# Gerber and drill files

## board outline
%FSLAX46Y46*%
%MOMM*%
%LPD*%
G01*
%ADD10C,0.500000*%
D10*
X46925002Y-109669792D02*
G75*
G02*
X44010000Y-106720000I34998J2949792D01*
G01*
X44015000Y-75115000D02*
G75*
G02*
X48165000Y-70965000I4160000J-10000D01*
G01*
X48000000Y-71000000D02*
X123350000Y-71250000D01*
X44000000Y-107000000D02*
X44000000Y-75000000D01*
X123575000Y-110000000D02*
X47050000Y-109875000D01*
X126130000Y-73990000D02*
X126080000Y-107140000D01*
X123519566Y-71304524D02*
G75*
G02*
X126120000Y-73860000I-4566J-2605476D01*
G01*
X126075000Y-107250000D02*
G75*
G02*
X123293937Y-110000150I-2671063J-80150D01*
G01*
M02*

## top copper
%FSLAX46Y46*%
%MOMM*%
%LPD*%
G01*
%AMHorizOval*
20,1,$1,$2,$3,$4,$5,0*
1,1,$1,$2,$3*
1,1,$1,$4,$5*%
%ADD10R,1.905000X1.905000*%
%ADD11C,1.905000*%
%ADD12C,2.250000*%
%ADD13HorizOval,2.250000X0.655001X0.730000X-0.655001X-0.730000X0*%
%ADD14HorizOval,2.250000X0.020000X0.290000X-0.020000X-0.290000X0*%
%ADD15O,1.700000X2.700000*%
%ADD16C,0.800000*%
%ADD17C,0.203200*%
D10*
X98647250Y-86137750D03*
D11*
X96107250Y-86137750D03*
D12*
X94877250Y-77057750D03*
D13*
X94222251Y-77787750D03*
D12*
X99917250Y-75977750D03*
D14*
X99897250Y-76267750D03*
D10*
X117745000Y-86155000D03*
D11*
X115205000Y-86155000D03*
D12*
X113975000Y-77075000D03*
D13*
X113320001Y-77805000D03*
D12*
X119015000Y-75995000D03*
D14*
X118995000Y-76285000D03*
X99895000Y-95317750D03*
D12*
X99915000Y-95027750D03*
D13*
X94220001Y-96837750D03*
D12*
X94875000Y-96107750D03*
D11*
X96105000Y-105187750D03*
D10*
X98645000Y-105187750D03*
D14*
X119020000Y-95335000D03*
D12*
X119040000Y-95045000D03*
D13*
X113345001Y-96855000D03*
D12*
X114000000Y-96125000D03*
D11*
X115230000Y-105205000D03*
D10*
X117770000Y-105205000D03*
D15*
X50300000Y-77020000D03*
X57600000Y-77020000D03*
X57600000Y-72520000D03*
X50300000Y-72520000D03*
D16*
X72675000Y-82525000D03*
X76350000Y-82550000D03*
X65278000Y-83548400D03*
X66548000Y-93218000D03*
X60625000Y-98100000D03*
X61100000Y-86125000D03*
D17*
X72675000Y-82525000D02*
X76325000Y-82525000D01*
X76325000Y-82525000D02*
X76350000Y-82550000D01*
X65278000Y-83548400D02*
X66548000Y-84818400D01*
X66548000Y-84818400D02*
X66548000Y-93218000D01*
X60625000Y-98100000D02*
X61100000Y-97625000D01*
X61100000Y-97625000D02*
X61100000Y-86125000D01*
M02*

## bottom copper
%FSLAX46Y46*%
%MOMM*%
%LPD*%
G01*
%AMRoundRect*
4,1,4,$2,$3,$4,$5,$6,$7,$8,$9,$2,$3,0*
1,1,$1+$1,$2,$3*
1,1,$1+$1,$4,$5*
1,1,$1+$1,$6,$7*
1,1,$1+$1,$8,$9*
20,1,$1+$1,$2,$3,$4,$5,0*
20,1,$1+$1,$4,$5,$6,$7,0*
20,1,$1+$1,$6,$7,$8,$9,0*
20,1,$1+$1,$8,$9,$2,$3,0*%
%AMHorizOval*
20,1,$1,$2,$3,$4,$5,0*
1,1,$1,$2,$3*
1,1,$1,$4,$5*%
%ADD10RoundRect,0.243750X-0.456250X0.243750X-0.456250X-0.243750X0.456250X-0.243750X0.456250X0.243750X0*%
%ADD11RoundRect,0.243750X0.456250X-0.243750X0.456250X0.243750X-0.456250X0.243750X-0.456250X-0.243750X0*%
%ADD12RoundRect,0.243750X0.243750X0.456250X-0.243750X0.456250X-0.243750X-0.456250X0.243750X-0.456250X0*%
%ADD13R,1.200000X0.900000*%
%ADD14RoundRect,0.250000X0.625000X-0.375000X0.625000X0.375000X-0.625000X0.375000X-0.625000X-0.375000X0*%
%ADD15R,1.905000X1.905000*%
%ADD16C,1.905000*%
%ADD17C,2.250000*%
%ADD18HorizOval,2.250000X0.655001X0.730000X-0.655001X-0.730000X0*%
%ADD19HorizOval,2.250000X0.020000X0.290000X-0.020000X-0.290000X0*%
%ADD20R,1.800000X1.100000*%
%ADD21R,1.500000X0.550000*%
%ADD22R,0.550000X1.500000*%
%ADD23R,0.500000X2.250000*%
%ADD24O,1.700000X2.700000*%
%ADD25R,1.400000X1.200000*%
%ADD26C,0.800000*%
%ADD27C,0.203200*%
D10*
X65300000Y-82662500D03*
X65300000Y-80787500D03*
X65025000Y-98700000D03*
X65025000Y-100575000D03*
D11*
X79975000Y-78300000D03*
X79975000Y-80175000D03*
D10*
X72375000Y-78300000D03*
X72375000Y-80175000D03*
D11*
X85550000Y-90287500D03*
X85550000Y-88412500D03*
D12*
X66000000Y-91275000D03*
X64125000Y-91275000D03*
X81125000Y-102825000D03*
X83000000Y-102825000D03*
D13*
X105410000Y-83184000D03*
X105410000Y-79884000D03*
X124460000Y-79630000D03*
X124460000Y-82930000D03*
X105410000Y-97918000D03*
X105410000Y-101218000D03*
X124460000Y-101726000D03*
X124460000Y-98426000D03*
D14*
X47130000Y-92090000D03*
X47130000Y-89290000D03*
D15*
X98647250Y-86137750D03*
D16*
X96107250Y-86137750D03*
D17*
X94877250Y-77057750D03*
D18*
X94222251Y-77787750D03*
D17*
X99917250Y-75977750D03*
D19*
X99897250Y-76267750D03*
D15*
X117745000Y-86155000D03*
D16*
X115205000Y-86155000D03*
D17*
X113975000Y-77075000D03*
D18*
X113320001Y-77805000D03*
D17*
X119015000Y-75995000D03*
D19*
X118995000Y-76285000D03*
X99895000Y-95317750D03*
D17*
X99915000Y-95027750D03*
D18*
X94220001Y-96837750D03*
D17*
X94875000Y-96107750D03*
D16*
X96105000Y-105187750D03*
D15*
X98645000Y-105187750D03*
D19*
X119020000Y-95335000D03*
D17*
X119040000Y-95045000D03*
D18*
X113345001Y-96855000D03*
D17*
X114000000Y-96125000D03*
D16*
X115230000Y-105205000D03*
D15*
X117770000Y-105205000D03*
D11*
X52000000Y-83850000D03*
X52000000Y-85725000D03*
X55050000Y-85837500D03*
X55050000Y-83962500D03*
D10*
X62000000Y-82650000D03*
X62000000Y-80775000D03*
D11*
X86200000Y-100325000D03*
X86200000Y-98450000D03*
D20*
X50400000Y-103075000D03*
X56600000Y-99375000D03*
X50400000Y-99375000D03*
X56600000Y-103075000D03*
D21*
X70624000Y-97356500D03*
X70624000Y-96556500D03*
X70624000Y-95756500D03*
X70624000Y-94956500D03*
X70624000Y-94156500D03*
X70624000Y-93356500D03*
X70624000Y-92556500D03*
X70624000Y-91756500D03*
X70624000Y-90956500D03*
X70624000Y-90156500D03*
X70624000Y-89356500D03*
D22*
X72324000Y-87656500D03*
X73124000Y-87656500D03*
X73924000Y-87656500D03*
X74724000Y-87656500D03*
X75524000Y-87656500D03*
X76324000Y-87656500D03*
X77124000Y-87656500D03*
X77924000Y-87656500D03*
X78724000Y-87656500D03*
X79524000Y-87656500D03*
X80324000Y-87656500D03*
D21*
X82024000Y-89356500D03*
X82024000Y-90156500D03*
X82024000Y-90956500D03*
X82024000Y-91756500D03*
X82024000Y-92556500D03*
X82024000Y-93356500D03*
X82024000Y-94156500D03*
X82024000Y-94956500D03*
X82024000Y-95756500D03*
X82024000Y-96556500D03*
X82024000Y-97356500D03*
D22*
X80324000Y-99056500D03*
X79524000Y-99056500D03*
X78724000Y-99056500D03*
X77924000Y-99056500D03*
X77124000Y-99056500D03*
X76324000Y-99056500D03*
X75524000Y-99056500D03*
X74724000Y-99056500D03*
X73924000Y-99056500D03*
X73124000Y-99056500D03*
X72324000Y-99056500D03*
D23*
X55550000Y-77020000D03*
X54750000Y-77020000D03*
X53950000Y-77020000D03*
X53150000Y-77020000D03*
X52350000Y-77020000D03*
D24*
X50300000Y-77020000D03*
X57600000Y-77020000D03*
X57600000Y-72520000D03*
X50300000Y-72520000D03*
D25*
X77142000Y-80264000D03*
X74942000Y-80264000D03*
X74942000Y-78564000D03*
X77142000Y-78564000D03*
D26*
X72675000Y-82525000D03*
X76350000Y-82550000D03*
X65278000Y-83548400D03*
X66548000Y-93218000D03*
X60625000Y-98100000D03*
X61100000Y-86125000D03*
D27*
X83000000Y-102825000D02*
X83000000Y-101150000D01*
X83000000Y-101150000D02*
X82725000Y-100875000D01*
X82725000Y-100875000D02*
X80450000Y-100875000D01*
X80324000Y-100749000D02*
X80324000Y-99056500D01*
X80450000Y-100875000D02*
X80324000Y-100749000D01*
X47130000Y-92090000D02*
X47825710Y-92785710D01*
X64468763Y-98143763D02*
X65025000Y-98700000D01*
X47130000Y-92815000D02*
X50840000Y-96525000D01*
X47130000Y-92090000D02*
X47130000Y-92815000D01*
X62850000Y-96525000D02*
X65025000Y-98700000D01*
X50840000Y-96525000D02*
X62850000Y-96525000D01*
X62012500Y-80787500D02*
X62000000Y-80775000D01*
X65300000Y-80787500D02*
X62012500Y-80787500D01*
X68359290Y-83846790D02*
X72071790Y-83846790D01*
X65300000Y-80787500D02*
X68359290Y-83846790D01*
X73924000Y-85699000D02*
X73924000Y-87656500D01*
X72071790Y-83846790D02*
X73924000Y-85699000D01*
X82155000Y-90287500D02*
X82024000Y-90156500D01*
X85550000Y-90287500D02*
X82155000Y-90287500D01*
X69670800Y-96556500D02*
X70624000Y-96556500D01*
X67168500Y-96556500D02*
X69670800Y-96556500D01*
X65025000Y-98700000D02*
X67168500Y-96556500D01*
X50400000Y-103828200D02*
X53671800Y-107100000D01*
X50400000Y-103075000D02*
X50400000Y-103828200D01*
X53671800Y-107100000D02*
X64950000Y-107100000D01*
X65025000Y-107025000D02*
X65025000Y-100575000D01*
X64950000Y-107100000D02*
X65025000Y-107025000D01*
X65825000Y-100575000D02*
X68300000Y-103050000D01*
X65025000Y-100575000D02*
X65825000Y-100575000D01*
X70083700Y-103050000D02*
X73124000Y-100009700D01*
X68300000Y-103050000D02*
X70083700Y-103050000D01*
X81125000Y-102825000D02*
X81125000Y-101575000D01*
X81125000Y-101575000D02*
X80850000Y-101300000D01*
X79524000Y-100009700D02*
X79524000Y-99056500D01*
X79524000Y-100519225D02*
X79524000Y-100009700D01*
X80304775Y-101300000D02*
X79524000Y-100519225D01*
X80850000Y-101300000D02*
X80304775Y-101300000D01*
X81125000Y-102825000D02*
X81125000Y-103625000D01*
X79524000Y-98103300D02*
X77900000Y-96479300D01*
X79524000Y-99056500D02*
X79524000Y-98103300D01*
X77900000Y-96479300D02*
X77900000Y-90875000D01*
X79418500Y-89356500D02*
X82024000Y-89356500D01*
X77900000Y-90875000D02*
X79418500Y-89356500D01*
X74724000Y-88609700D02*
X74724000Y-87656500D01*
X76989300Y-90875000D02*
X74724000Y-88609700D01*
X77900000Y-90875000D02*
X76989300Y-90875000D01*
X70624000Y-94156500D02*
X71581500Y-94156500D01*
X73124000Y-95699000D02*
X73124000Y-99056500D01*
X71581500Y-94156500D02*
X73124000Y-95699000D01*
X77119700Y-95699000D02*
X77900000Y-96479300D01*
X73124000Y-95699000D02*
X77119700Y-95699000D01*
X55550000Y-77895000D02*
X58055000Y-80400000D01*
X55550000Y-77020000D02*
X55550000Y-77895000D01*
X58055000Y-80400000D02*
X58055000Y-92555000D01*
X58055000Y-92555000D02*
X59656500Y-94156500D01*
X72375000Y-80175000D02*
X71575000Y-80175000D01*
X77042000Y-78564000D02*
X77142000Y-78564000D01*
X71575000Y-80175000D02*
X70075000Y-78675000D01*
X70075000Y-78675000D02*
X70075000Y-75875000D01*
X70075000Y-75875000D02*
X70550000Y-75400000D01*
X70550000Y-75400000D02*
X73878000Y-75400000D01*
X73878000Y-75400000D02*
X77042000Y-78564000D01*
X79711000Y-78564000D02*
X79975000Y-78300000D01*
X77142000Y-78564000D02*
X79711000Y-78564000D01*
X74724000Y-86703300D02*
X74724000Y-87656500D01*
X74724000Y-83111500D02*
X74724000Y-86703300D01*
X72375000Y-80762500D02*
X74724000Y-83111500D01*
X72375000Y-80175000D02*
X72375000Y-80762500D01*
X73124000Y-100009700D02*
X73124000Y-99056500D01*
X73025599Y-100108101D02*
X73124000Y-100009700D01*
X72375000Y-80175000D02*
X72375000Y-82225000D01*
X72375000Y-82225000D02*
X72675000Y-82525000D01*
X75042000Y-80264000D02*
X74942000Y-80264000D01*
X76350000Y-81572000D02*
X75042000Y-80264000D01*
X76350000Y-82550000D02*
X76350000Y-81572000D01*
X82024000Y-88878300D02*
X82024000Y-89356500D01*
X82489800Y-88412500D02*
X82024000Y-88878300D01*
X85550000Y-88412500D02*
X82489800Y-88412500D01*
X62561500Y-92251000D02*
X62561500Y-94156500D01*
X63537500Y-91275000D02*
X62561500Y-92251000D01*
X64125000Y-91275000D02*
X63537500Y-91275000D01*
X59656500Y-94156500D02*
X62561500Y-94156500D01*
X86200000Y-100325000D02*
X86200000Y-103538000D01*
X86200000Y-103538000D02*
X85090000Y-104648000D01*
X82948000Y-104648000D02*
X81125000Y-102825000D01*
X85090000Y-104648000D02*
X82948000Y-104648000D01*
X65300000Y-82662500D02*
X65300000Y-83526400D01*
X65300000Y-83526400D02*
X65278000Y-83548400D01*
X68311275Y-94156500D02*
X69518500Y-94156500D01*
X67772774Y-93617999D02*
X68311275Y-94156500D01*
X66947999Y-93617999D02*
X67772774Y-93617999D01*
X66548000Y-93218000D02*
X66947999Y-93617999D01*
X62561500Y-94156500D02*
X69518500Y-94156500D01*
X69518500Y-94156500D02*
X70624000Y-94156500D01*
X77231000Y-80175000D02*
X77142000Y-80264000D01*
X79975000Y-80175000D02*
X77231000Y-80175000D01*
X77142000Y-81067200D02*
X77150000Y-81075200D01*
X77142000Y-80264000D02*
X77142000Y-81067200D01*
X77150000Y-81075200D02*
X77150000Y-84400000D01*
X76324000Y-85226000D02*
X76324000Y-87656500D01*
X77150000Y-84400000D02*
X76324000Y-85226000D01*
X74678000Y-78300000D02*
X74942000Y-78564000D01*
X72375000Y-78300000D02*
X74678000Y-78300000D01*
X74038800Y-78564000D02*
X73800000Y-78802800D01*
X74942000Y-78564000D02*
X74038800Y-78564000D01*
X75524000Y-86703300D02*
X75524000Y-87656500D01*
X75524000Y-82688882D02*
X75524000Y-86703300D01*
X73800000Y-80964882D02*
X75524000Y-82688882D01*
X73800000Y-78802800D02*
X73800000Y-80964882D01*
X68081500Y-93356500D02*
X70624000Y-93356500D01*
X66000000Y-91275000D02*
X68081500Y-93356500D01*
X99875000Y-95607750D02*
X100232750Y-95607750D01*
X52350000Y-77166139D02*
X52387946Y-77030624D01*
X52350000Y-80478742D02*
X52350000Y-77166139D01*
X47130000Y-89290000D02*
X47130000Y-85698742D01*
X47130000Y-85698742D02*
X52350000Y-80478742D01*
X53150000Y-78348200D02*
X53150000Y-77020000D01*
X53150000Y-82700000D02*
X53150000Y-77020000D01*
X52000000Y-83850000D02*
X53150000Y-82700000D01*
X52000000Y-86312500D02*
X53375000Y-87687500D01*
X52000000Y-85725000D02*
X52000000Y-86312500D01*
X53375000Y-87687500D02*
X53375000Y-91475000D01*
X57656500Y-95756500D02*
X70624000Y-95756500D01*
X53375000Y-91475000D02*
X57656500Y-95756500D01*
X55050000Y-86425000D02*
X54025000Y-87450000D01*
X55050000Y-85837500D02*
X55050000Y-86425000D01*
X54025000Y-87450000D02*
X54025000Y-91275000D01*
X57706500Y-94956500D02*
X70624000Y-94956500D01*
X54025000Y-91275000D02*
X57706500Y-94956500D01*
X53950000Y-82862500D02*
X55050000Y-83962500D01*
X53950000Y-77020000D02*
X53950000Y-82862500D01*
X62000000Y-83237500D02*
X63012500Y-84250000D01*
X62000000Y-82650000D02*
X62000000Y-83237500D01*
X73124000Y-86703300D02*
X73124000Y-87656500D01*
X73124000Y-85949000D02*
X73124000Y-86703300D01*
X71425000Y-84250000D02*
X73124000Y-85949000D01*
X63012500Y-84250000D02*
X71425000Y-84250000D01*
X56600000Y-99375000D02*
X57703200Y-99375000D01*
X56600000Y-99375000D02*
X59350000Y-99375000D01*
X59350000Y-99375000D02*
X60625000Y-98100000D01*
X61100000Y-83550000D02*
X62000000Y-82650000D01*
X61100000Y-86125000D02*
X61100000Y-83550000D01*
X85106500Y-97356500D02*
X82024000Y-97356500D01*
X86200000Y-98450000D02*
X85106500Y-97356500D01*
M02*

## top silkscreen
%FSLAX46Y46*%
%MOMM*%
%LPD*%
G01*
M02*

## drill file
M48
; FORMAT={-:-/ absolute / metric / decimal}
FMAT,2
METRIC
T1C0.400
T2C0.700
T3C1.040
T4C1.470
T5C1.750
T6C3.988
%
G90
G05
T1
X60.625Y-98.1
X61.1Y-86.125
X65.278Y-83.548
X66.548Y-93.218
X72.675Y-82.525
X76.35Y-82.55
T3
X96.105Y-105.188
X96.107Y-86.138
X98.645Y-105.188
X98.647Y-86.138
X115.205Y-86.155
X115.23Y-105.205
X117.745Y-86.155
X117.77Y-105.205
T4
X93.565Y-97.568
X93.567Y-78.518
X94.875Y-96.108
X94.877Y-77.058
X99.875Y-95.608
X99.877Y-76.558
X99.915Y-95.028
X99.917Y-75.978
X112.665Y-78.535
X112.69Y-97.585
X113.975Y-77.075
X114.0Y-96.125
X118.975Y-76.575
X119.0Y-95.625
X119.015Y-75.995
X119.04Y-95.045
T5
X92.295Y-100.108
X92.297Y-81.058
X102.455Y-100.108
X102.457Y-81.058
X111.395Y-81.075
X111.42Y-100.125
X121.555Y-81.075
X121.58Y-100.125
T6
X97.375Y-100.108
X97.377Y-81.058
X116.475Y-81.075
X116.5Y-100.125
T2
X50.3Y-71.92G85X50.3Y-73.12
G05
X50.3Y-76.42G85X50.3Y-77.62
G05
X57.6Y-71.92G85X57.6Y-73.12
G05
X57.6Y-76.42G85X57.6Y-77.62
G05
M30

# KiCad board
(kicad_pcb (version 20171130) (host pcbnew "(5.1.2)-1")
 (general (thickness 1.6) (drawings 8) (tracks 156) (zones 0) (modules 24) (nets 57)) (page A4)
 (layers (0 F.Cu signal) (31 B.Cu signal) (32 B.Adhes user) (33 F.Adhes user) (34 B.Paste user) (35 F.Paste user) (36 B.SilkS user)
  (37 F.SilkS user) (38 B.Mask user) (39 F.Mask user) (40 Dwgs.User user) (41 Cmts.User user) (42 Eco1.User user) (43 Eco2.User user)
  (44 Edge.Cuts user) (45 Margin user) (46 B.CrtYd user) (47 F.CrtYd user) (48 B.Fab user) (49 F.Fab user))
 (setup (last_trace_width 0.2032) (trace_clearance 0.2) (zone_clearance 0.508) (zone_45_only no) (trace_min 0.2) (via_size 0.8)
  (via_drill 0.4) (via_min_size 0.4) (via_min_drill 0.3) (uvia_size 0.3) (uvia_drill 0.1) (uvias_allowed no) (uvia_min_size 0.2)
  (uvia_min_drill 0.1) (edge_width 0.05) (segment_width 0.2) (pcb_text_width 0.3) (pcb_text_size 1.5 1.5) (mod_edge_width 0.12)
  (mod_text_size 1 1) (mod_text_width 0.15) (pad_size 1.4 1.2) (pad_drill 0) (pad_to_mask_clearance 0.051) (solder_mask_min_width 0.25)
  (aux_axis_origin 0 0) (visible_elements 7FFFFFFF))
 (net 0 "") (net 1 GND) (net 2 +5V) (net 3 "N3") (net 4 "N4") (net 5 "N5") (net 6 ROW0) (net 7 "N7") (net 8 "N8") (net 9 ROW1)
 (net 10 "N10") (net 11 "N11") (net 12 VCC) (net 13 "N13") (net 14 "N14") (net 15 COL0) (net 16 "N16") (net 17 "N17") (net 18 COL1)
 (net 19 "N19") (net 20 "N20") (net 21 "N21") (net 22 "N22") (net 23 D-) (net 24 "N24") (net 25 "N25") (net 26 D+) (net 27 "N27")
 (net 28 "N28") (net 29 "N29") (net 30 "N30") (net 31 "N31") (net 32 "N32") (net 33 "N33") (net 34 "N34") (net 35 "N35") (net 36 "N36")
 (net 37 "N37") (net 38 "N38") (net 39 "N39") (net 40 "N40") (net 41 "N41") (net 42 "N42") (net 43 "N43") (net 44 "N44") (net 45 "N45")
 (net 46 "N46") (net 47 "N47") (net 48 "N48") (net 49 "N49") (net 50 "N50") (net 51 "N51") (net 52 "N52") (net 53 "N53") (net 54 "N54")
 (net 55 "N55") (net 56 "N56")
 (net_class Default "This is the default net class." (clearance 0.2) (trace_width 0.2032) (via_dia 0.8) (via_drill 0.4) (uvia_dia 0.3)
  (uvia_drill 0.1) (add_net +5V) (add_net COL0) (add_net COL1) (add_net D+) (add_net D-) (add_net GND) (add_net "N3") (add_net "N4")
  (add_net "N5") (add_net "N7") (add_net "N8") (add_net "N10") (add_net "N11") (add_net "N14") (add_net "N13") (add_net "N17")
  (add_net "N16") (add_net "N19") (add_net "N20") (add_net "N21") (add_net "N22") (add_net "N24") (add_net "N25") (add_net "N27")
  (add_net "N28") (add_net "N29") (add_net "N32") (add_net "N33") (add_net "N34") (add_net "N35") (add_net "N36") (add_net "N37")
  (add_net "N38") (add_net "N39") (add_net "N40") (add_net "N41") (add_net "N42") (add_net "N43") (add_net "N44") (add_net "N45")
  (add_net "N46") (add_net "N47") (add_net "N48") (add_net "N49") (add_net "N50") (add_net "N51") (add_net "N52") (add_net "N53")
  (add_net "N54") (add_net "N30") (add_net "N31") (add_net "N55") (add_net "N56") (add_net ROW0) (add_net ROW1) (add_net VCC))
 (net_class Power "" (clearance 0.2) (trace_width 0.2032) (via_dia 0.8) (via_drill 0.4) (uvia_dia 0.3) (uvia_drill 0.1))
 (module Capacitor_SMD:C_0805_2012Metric (layer B.Cu) (at 65.3 81.725 270)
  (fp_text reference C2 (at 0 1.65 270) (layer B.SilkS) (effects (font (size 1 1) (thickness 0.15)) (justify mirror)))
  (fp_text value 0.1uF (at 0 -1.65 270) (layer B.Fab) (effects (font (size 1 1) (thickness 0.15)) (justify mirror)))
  (pad 2 smd roundrect (at 0.9375 0 270) (size 0.975 1.4) (layers B.Cu B.Paste B.Mask) (roundrect_rratio 0.25) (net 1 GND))
  (pad 1 smd roundrect (at -0.9375 0 270) (size 0.975 1.4) (layers B.Cu B.Paste B.Mask) (roundrect_rratio 0.25) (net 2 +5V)))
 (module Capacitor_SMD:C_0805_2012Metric (layer B.Cu) (at 65.025 99.6375 270)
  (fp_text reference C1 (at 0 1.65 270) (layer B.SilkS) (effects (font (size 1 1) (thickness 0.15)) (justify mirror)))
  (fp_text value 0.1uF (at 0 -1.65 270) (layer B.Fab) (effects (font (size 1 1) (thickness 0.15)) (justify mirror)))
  (pad 1 smd roundrect (at -0.9375 0 270) (size 0.975 1.4) (layers B.Cu B.Paste B.Mask) (roundrect_rratio 0.25) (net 2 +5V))
  (pad 2 smd roundrect (at 0.9375 0 270) (size 0.975 1.4) (layers B.Cu B.Paste B.Mask) (roundrect_rratio 0.25) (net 1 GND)))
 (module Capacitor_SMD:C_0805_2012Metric (layer B.Cu) (at 79.975 79.2375 90)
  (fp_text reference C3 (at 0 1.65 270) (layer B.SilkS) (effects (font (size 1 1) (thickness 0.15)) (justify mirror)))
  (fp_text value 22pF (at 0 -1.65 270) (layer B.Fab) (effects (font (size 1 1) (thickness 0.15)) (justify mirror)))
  (pad 2 smd roundrect (at 0.9375 0 90) (size 0.975 1.4) (layers B.Cu B.Paste B.Mask) (roundrect_rratio 0.25) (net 1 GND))
  (pad 1 smd roundrect (at -0.9375 0 90) (size 0.975 1.4) (layers B.Cu B.Paste B.Mask) (roundrect_rratio 0.25) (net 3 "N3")))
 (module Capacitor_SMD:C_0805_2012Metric (layer B.Cu) (at 72.375 79.2375 270)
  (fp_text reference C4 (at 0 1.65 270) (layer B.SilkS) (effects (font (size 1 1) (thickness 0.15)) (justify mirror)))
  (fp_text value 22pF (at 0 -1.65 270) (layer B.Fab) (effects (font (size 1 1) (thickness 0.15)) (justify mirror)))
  (pad 1 smd roundrect (at -0.9375 0 270) (size 0.975 1.4) (layers B.Cu B.Paste B.Mask) (roundrect_rratio 0.25) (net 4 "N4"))
  (pad 2 smd roundrect (at 0.9375 0 270) (size 0.975 1.4) (layers B.Cu B.Paste B.Mask) (roundrect_rratio 0.25) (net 1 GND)))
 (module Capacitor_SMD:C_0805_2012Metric (layer B.Cu) (at 85.55 89.35 90)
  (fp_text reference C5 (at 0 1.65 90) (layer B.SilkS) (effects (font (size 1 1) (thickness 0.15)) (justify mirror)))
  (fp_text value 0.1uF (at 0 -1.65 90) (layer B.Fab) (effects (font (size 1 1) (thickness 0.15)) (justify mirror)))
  (pad 1 smd roundrect (at -0.9375 0 90) (size 0.975 1.4) (layers B.Cu B.Paste B.Mask) (roundrect_rratio 0.25) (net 2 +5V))
  (pad 2 smd roundrect (at 0.9375 0 90) (size 0.975 1.4) (layers B.Cu B.Paste B.Mask) (roundrect_rratio 0.25) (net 1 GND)))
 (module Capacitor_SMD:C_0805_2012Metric (layer B.Cu) (at 65.0625 91.275 180)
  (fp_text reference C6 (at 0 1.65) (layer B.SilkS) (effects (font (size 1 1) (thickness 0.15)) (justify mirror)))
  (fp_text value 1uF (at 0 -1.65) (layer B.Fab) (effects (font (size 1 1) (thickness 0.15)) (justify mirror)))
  (pad 1 smd roundrect (at -0.9375 0 180) (size 0.975 1.4) (layers B.Cu B.Paste B.Mask) (roundrect_rratio 0.25) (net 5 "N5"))
  (pad 2 smd roundrect (at 0.9375 0 180) (size 0.975 1.4) (layers B.Cu B.Paste B.Mask) (roundrect_rratio 0.25) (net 1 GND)))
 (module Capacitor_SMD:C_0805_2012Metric (layer B.Cu) (at 82.0625 102.825 180)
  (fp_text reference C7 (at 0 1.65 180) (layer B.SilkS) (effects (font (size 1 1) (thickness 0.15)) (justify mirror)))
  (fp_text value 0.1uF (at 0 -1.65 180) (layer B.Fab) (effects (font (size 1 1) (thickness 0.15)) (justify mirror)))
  (pad 2 smd roundrect (at 0.9375 0 180) (size 0.975 1.4) (layers B.Cu B.Paste B.Mask) (roundrect_rratio 0.25) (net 1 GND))
  (pad 1 smd roundrect (at -0.9375 0 180) (size 0.975 1.4) (layers B.Cu B.Paste B.Mask) (roundrect_rratio 0.25) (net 2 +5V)))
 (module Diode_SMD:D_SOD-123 (layer B.Cu) (at 105.41 81.534 90)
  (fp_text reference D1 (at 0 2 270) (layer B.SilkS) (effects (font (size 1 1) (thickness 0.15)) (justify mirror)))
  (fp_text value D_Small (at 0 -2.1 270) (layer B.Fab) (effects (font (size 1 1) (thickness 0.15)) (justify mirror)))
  (pad 1 smd rect (at -1.65 0 90) (size 0.9 1.2) (layers B.Cu B.Paste B.Mask) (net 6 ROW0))
  (pad 2 smd rect (at 1.65 0 90) (size 0.9 1.2) (layers B.Cu B.Paste B.Mask) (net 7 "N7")))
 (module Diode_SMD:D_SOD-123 (layer B.Cu) (at 124.46 81.28 90)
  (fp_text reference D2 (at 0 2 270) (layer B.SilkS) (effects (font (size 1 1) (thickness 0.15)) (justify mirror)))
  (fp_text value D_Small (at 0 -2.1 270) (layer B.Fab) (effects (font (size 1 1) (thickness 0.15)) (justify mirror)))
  (pad 2 smd rect (at 1.65 0 90) (size 0.9 1.2) (layers B.Cu B.Paste B.Mask) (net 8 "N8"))
  (pad 1 smd rect (at -1.65 0 90) (size 0.9 1.2) (layers B.Cu B.Paste B.Mask) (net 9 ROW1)))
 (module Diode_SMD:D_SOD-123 (layer B.Cu) (at 105.41 99.568 270)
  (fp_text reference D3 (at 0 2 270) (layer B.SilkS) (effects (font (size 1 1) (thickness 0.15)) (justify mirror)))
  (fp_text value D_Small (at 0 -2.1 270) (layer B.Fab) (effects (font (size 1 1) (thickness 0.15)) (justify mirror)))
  (pad 1 smd rect (at -1.65 0 270) (size 0.9 1.2) (layers B.Cu B.Paste B.Mask) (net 6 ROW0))
  (pad 2 smd rect (at 1.65 0 270) (size 0.9 1.2) (layers B.Cu B.Paste B.Mask) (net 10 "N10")))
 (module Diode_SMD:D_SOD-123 (layer B.Cu) (at 124.46 100.076 270)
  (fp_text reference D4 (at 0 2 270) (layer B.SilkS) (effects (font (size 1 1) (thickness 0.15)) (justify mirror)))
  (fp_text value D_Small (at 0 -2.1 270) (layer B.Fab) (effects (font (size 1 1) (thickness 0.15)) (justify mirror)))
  (pad 2 smd rect (at 1.65 0 270) (size 0.9 1.2) (layers B.Cu B.Paste B.Mask) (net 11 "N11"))
  (pad 1 smd rect (at -1.65 0 270) (size 0.9 1.2) (layers B.Cu B.Paste B.Mask) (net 9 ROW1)))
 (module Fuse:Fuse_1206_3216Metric (layer B.Cu) (at 47.13 90.69 90)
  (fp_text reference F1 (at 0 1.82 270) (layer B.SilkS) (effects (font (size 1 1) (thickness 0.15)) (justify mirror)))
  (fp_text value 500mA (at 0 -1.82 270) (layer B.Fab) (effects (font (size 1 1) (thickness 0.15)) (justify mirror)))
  (pad 1 smd roundrect (at -1.4 0 90) (size 1.25 1.75) (layers B.Cu B.Paste B.Mask) (roundrect_rratio 0.2) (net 2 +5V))
  (pad 2 smd roundrect (at 1.4 0 90) (size 1.25 1.75) (layers B.Cu B.Paste B.Mask) (roundrect_rratio 0.2) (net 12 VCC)))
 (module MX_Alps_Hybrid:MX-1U (layer F.Cu) (at 97.37725 81.05775)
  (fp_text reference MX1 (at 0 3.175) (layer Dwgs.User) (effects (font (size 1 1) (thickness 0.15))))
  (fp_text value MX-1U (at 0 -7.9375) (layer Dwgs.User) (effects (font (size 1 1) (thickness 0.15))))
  (pad "" np_thru_hole circle (at 5.08 0 48.0996) (size 1.75 1.75) (drill 1.75) (layers *.Cu *.Mask))
  (pad "" np_thru_hole circle (at -5.08 0 48.0996) (size 1.75 1.75) (drill 1.75) (layers *.Cu *.Mask))
  (pad 4 thru_hole rect (at 1.27 5.08) (size 1.905 1.905) (drill 1.04) (layers *.Cu B.Mask) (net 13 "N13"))
  (pad 3 thru_hole circle (at -1.27 5.08) (size 1.905 1.905) (drill 1.04) (layers *.Cu B.Mask) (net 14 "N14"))
  (pad 1 thru_hole circle (at -2.5 -4) (size 2.25 2.25) (drill 1.47) (layers *.Cu B.Mask) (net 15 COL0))
  (pad "" np_thru_hole circle (at 0 0) (size 3.9878 3.9878) (drill 3.9878) (layers *.Cu *.Mask))
  (pad 1 thru_hole oval (at -3.81 -2.54 48.0996) (size 4.211556 2.25) (drill 1.47 (offset 0.980778 0)) (layers *.Cu B.Mask) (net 15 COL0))
  (pad 2 thru_hole circle (at 2.54 -5.08) (size 2.25 2.25) (drill 1.47) (layers *.Cu B.Mask) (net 7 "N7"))
  (pad 2 thru_hole oval (at 2.5 -4.5 86.0548) (size 2.831378 2.25) (drill 1.47 (offset 0.290689 0)) (layers *.Cu B.Mask) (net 7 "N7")))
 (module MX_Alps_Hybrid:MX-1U (layer F.Cu) (at 116.475 81.075)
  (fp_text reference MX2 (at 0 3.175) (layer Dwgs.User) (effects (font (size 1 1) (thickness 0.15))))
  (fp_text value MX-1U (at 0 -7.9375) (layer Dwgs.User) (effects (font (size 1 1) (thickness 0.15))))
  (pad "" np_thru_hole circle (at 5.08 0 48.0996) (size 1.75 1.75) (drill 1.75) (layers *.Cu *.Mask))
  (pad "" np_thru_hole circle (at -5.08 0 48.0996) (size 1.75 1.75) (drill 1.75) (layers *.Cu *.Mask))
  (pad 4 thru_hole rect (at 1.27 5.08) (size 1.905 1.905) (drill 1.04) (layers *.Cu B.Mask) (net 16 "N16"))
  (pad 3 thru_hole circle (at -1.27 5.08) (size 1.905 1.905) (drill 1.04) (layers *.Cu B.Mask) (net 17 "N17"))
  (pad 1 thru_hole circle (at -2.5 -4) (size 2.25 2.25) (drill 1.47) (layers *.Cu B.Mask) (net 15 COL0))
  (pad "" np_thru_hole circle (at 0 0) (size 3.9878 3.9878) (drill 3.9878) (layers *.Cu *.Mask))
  (pad 1 thru_hole oval (at -3.81 -2.54 48.0996) (size 4.211556 2.25) (drill 1.47 (offset 0.980778 0)) (layers *.Cu B.Mask) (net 15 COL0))
  (pad 2 thru_hole circle (at 2.54 -5.08) (size 2.25 2.25) (drill 1.47) (layers *.Cu B.Mask) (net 8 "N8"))
  (pad 2 thru_hole oval (at 2.5 -4.5 86.0548) (size 2.831378 2.25) (drill 1.47 (offset 0.290689 0)) (layers *.Cu B.Mask) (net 8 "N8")))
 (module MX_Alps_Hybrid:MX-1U (layer F.Cu) (at 97.375 100.10775)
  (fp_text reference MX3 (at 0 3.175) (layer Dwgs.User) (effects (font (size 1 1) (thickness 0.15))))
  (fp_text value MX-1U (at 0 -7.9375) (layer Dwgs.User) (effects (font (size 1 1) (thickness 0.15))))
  (pad 2 thru_hole oval (at 2.5 -4.5 86.0548) (size 2.831378 2.25) (drill 1.47 (offset 0.290689 0)) (layers *.Cu B.Mask) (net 10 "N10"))
  (pad 2 thru_hole circle (at 2.54 -5.08) (size 2.25 2.25) (drill 1.47) (layers *.Cu B.Mask) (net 10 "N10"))
  (pad 1 thru_hole oval (at -3.81 -2.54 48.0996) (size 4.211556 2.25) (drill 1.47 (offset 0.980778 0)) (layers *.Cu B.Mask) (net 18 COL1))
  (pad "" np_thru_hole circle (at 0 0) (size 3.9878 3.9878) (drill 3.9878) (layers *.Cu *.Mask))
  (pad 1 thru_hole circle (at -2.5 -4) (size 2.25 2.25) (drill 1.47) (layers *.Cu B.Mask) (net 18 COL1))
  (pad 3 thru_hole circle (at -1.27 5.08) (size 1.905 1.905) (drill 1.04) (layers *.Cu B.Mask) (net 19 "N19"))
  (pad 4 thru_hole rect (at 1.27 5.08) (size 1.905 1.905) (drill 1.04) (layers *.Cu B.Mask) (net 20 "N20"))
  (pad "" np_thru_hole circle (at -5.08 0 48.0996) (size 1.75 1.75) (drill 1.75) (layers *.Cu *.Mask))
  (pad "" np_thru_hole circle (at 5.08 0 48.0996) (size 1.75 1.75) (drill 1.75) (layers *.Cu *.Mask)))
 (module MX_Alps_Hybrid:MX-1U (layer F.Cu) (at 116.5 100.125)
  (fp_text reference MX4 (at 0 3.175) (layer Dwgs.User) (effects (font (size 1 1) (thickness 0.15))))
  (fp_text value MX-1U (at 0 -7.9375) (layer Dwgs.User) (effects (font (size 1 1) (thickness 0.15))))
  (pad 2 thru_hole oval (at 2.5 -4.5 86.0548) (size 2.831378 2.25) (drill 1.47 (offset 0.290689 0)) (layers *.Cu B.Mask) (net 11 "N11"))
  (pad 2 thru_hole circle (at 2.54 -5.08) (size 2.25 2.25) (drill 1.47) (layers *.Cu B.Mask) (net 11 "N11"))
  (pad 1 thru_hole oval (at -3.81 -2.54 48.0996) (size 4.211556 2.25) (drill 1.47 (offset 0.980778 0)) (layers *.Cu B.Mask) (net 18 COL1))
  (pad "" np_thru_hole circle (at 0 0) (size 3.9878 3.9878) (drill 3.9878) (layers *.Cu *.Mask))
  (pad 1 thru_hole circle (at -2.5 -4) (size 2.25 2.25) (drill 1.47) (layers *.Cu B.Mask) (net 18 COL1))
  (pad 3 thru_hole circle (at -1.27 5.08) (size 1.905 1.905) (drill 1.04) (layers *.Cu B.Mask) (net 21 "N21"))
  (pad 4 thru_hole rect (at 1.27 5.08) (size 1.905 1.905) (drill 1.04) (layers *.Cu B.Mask) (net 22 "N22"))
  (pad "" np_thru_hole circle (at -5.08 0 48.0996) (size 1.75 1.75) (drill 1.75) (layers *.Cu *.Mask))
  (pad "" np_thru_hole circle (at 5.08 0 48.0996) (size 1.75 1.75) (drill 1.75) (layers *.Cu *.Mask)))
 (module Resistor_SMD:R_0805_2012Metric (layer B.Cu) (at 52 84.7875 90)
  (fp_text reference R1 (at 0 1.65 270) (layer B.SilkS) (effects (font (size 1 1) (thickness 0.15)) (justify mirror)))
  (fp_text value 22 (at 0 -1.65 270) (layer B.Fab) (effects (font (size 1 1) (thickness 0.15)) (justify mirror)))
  (pad 2 smd roundrect (at 0.9375 0 90) (size 0.975 1.4) (layers B.Cu B.Paste B.Mask) (roundrect_rratio 0.25) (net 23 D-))
  (pad 1 smd roundrect (at -0.9375 0 90) (size 0.975 1.4) (layers B.Cu B.Paste B.Mask) (roundrect_rratio 0.25) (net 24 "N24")))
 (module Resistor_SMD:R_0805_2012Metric (layer B.Cu) (at 55.05 84.9 90)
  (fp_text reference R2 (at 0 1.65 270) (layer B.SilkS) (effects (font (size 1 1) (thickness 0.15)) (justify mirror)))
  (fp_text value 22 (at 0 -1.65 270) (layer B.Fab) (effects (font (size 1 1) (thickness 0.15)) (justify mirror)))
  (pad 1 smd roundrect (at -0.9375 0 90) (size 0.975 1.4) (layers B.Cu B.Paste B.Mask) (roundrect_rratio 0.25) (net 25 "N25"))
  (pad 2 smd roundrect (at 0.9375 0 90) (size 0.975 1.4) (layers B.Cu B.Paste B.Mask) (roundrect_rratio 0.25) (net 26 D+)))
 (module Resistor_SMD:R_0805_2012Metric (layer B.Cu) (at 62 81.7125 270)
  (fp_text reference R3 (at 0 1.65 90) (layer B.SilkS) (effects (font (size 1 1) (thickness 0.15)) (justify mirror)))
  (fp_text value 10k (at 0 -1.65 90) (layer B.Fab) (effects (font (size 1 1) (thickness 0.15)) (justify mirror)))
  (pad 2 smd roundrect (at 0.9375 0 270) (size 0.975 1.4) (layers B.Cu B.Paste B.Mask) (roundrect_rratio 0.25) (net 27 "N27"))
  (pad 1 smd roundrect (at -0.9375 0 270) (size 0.975 1.4) (layers B.Cu B.Paste B.Mask) (roundrect_rratio 0.25) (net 2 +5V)))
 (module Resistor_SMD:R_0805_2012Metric (layer B.Cu) (at 86.2 99.3875 90)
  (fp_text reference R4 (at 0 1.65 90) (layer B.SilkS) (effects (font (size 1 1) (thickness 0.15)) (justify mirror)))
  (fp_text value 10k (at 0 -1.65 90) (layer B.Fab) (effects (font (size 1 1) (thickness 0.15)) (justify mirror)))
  (pad 1 smd roundrect (at -0.9375 0 90) (size 0.975 1.4) (layers B.Cu B.Paste B.Mask) (roundrect_rratio 0.25) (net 1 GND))
  (pad 2 smd roundrect (at 0.9375 0 90) (size 0.975 1.4) (layers B.Cu B.Paste B.Mask) (roundrect_rratio 0.25) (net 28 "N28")))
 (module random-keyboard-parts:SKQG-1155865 (layer B.Cu) (at 53.5 101.225 180)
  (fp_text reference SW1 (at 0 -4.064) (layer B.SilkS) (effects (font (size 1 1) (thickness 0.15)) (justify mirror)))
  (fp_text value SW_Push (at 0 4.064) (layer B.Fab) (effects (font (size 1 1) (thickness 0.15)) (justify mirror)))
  (pad 1 smd rect (at 3.1 -1.85 180) (size 1.8 1.1) (layers B.Cu B.Paste B.Mask) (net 1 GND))
  (pad 2 smd rect (at -3.1 1.85 180) (size 1.8 1.1) (layers B.Cu B.Paste B.Mask) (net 27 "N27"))
  (pad 3 smd rect (at 3.1 1.85 180) (size 1.8 1.1) (layers B.Cu B.Paste B.Mask))
  (pad 4 smd rect (at -3.1 -1.85 180) (size 1.8 1.1) (layers B.Cu B.Paste B.Mask)))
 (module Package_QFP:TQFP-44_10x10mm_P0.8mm (layer B.Cu) (at 76.324 93.3565)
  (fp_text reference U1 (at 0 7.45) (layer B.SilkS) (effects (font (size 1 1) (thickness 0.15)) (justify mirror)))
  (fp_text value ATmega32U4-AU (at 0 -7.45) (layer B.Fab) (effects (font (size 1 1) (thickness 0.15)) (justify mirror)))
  (pad 1 smd rect (at -5.7 4) (size 1.5 0.55) (layers B.Cu B.Paste B.Mask) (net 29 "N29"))
  (pad 2 smd rect (at -5.7 3.2) (size 1.5 0.55) (layers B.Cu B.Paste B.Mask) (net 2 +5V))
  (pad 3 smd rect (at -5.7 2.4) (size 1.5 0.55) (layers B.Cu B.Paste B.Mask) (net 24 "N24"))
  (pad 4 smd rect (at -5.7 1.6) (size 1.5 0.55) (layers B.Cu B.Paste B.Mask) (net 25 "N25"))
  (pad 5 smd rect (at -5.7 0.8) (size 1.5 0.55) (layers B.Cu B.Paste B.Mask) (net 1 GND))
  (pad 6 smd rect (at -5.7 0) (size 1.5 0.55) (layers B.Cu B.Paste B.Mask) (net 5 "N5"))
  (pad 7 smd rect (at -5.7 -0.8) (size 1.5 0.55) (layers B.Cu B.Paste B.Mask) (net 2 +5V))
  (pad 8 smd rect (at -5.7 -1.6) (size 1.5 0.55) (layers B.Cu B.Paste B.Mask) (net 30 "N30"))
  (pad 9 smd rect (at -5.7 -2.4) (size 1.5 0.55) (layers B.Cu B.Paste B.Mask) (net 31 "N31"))
  (pad 10 smd rect (at -5.7 -3.2) (size 1.5 0.55) (layers B.Cu B.Paste B.Mask) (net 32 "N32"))
  (pad 11 smd rect (at -5.7 -4) (size 1.5 0.55) (layers B.Cu B.Paste B.Mask) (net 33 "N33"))
  (pad 12 smd rect (at -4 -5.7 270) (size 1.5 0.55) (layers B.Cu B.Paste B.Mask) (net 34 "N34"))
  (pad 13 smd rect (at -3.2 -5.7 270) (size 1.5 0.55) (layers B.Cu B.Paste B.Mask) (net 27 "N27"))
  (pad 14 smd rect (at -2.4 -5.7 270) (size 1.5 0.55) (layers B.Cu B.Paste B.Mask) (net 2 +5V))
  (pad 15 smd rect (at -1.6 -5.7 270) (size 1.5 0.55) (layers B.Cu B.Paste B.Mask) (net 1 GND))
  (pad 16 smd rect (at -0.8 -5.7 270) (size 1.5 0.55) (layers B.Cu B.Paste B.Mask) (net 4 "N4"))
  (pad 17 smd rect (at 0 -5.7 270) (size 1.5 0.55) (layers B.Cu B.Paste B.Mask) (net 3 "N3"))
  (pad 18 smd rect (at 0.8 -5.7 270) (size 1.5 0.55) (layers B.Cu B.Paste B.Mask) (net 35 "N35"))
  (pad 19 smd rect (at 1.6 -5.7 270) (size 1.5 0.55) (layers B.Cu B.Paste B.Mask) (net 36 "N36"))
  (pad 20 smd rect (at 2.4 -5.7 270) (size 1.5 0.55) (layers B.Cu B.Paste B.Mask) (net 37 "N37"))
  (pad 21 smd rect (at 3.2 -5.7 270) (size 1.5 0.55) (layers B.Cu B.Paste B.Mask) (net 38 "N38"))
  (pad 22 smd rect (at 4 -5.7 270) (size 1.5 0.55) (layers B.Cu B.Paste B.Mask) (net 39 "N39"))
  (pad 23 smd rect (at 5.7 -4) (size 1.5 0.55) (layers B.Cu B.Paste B.Mask) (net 1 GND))
  (pad 24 smd rect (at 5.7 -3.2) (size 1.5 0.55) (layers B.Cu B.Paste B.Mask) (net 2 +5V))
  (pad 25 smd rect (at 5.7 -2.4) (size 1.5 0.55) (layers B.Cu B.Paste B.Mask) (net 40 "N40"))
  (pad 26 smd rect (at 5.7 -1.6) (size 1.5 0.55) (layers B.Cu B.Paste B.Mask) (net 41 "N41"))
  (pad 27 smd rect (at 5.7 -0.8) (size 1.5 0.55) (layers B.Cu B.Paste B.Mask) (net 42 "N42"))
  (pad 28 smd rect (at 5.7 0) (size 1.5 0.55) (layers B.Cu B.Paste B.Mask) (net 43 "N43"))
  (pad 29 smd rect (at 5.7 0.8) (size 1.5 0.55) (layers B.Cu B.Paste B.Mask) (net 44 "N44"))
  (pad 30 smd rect (at 5.7 1.6) (size 1.5 0.55) (layers B.Cu B.Paste B.Mask) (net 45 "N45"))
  (pad 31 smd rect (at 5.7 2.4) (size 1.5 0.55) (layers B.Cu B.Paste B.Mask) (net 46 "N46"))
  (pad 32 smd rect (at 5.7 3.2) (size 1.5 0.55) (layers B.Cu B.Paste B.Mask) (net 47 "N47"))
  (pad 33 smd rect (at 5.7 4) (size 1.5 0.55) (layers B.Cu B.Paste B.Mask) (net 28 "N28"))
  (pad 34 smd rect (at 4 5.7 270) (size 1.5 0.55) (layers B.Cu B.Paste B.Mask) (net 2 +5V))
  (pad 35 smd rect (at 3.2 5.7 270) (size 1.5 0.55) (layers B.Cu B.Paste B.Mask) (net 1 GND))
  (pad 36 smd rect (at 2.4 5.7 270) (size 1.5 0.55) (layers B.Cu B.Paste B.Mask) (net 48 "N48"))
  (pad 37 smd rect (at 1.6 5.7 270) (size 1.5 0.55) (layers B.Cu B.Paste B.Mask) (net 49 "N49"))
  (pad 38 smd rect (at 0.8 5.7 270) (size 1.5 0.55) (layers B.Cu B.Paste B.Mask) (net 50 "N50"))
  (pad 39 smd rect (at 0 5.7 270) (size 1.5 0.55) (layers B.Cu B.Paste B.Mask) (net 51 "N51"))
  (pad 40 smd rect (at -0.8 5.7 270) (size 1.5 0.55) (layers B.Cu B.Paste B.Mask) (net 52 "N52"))
  (pad 41 smd rect (at -1.6 5.7 270) (size 1.5 0.55) (layers B.Cu B.Paste B.Mask) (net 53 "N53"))
  (pad 42 smd rect (at -2.4 5.7 270) (size 1.5 0.55) (layers B.Cu B.Paste B.Mask) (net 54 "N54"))
  (pad 43 smd rect (at -3.2 5.7 270) (size 1.5 0.55) (layers B.Cu B.Paste B.Mask) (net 1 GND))
  (pad 44 smd rect (at -4 5.7 270) (size 1.5 0.55) (layers B.Cu B.Paste B.Mask) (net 2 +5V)))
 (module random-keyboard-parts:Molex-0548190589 (layer B.Cu) (at 53.95 72.52 270)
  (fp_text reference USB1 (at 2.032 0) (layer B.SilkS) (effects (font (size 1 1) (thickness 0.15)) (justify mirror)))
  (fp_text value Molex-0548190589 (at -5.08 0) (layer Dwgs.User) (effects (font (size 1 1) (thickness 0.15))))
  (pad 1 smd rect (at 4.5 -1.6 270) (size 2.25 0.5) (layers B.Cu B.Paste B.Mask) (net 1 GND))
  (pad 2 smd rect (at 4.5 -0.8 270) (size 2.25 0.5) (layers B.Cu B.Paste B.Mask) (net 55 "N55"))
  (pad 3 smd rect (at 4.5 0 270) (size 2.25 0.5) (layers B.Cu B.Paste B.Mask) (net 26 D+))
  (pad 4 smd rect (at 4.5 0.8 270) (size 2.25 0.5) (layers B.Cu B.Paste B.Mask) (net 23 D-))
  (pad 5 smd rect (at 4.5 1.6 270) (size 2.25 0.5) (layers B.Cu B.Paste B.Mask) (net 12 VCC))
  (pad 6 thru_hole oval (at 4.5 3.65 270) (size 2.7 1.7) (drill oval 1.9 0.7) (layers *.Cu *.Mask) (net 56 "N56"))
  (pad 6 thru_hole oval (at 4.5 -3.65 270) (size 2.7 1.7) (drill oval 1.9 0.7) (layers *.Cu *.Mask) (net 56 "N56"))
  (pad 6 thru_hole oval (at 0 -3.65 270) (size 2.7 1.7) (drill oval 1.9 0.7) (layers *.Cu *.Mask) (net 56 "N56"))
  (pad 6 thru_hole oval (at 0 3.65 270) (size 2.7 1.7) (drill oval 1.9 0.7) (layers *.Cu *.Mask) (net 56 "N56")))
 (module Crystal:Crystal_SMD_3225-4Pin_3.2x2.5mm (layer B.Cu) (at 76.042 79.414 180)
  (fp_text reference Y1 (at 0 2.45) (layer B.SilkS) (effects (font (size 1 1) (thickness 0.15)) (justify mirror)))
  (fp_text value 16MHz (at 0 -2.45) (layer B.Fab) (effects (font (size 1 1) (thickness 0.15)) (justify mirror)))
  (pad 1 smd rect (at -1.1 -0.85 180) (size 1.4 1.2) (layers B.Cu B.Paste B.Mask) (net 3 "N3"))
  (pad 2 smd rect (at 1.1 -0.85 180) (size 1.4 1.2) (layers B.Cu B.Paste B.Mask) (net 1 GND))
  (pad 3 smd rect (at 1.1 0.85 180) (size 1.4 1.2) (layers B.Cu B.Paste B.Mask) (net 4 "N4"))
  (pad 4 smd rect (at -1.1 0.85 180) (size 1.4 1.2) (layers B.Cu B.Paste B.Mask) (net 1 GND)))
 (gr_arc (start 46.96 106.72) (end 44.01 106.72) (angle -89.32023579) (layer Edge.Cuts) (width 0.5))
 (gr_arc (start 48.175 75.125) (end 48.165 70.965) (angle -89.72454005) (layer Edge.Cuts) (width 0.5))
 (gr_line (start 48 71) (end 123.35 71.25) (layer Edge.Cuts) (width 0.5))
 (gr_line (start 44 107) (end 44 75) (layer Edge.Cuts) (width 0.5))
 (gr_line (start 123.575 110) (end 47.05 109.875) (layer Edge.Cuts) (width 0.5))
 (gr_line (start 126.13 73.99) (end 126.08 107.14) (layer Edge.Cuts) (width 0.5))
 (gr_arc (start 123.515 73.91) (end 126.12 73.86) (angle -88.8) (layer Edge.Cuts) (width 0.5))
 (gr_arc (start 123.403937 107.33015) (end 123.293937 110.00015) (angle -94.07790525) (layer Edge.Cuts) (width 0.5))
 (segment (start 83 102.825) (end 83 101.15) (width 0.2032) (layer B.Cu) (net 2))
 (segment (start 83 101.15) (end 82.725 100.875) (width 0.2032) (layer B.Cu) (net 2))
 (segment (start 82.725 100.875) (end 80.45 100.875) (width 0.2032) (layer B.Cu) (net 2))
 (segment (start 80.324 100.749) (end 80.324 99.0565) (width 0.2032) (layer B.Cu) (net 2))
 (segment (start 80.45 100.875) (end 80.324 100.749) (width 0.2032) (layer B.Cu) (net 2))
 (segment (start 47.13 92.09) (end 47.82571 92.78571) (width 0.2032) (layer B.Cu) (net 2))
 (segment (start 64.468763 98.143763) (end 65.025 98.7) (width 0.2032) (layer B.Cu) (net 2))
 (segment (start 47.13 92.815) (end 50.84 96.525) (width 0.2032) (layer B.Cu) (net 2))
 (segment (start 47.13 92.09) (end 47.13 92.815) (width 0.2032) (layer B.Cu) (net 2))
 (segment (start 62.85 96.525) (end 65.025 98.7) (width 0.2032) (layer B.Cu) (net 2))
 (segment (start 50.84 96.525) (end 62.85 96.525) (width 0.2032) (layer B.Cu) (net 2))
 (segment (start 62.0125 80.7875) (end 62 80.775) (width 0.2032) (layer B.Cu) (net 2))
 (segment (start 65.3 80.7875) (end 62.0125 80.7875) (width 0.2032) (layer B.Cu) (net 2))
 (segment (start 68.35929 83.84679) (end 72.07179 83.84679) (width 0.2032) (layer B.Cu) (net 2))
 (segment (start 65.3 80.7875) (end 68.35929 83.84679) (width 0.2032) (layer B.Cu) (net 2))
 (segment (start 73.924 85.699) (end 73.924 87.6565) (width 0.2032) (layer B.Cu) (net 2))
 (segment (start 72.07179 83.84679) (end 73.924 85.699) (width 0.2032) (layer B.Cu) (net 2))
 (segment (start 82.155 90.2875) (end 82.024 90.1565) (width 0.2032) (layer B.Cu) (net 2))
 (segment (start 85.55 90.2875) (end 82.155 90.2875) (width 0.2032) (layer B.Cu) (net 2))
 (segment (start 69.6708 96.5565) (end 70.624 96.5565) (width 0.2032) (layer B.Cu) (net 2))
 (segment (start 67.1685 96.5565) (end 69.6708 96.5565) (width 0.2032) (layer B.Cu) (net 2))
 (segment (start 65.025 98.7) (end 67.1685 96.5565) (width 0.2032) (layer B.Cu) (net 2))
 (segment (start 50.4 103.8282) (end 53.6718 107.1) (width 0.2032) (layer B.Cu) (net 1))
 (segment (start 50.4 103.075) (end 50.4 103.8282) (width 0.2032) (layer B.Cu) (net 1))
 (segment (start 53.6718 107.1) (end 64.95 107.1) (width 0.2032) (layer B.Cu) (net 1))
 (segment (start 65.025 107.025) (end 65.025 100.575) (width 0.2032) (layer B.Cu) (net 1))
 (segment (start 64.95 107.1) (end 65.025 107.025) (width 0.2032) (layer B.Cu) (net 1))
 (segment (start 65.825 100.575) (end 68.3 103.05) (width 0.2032) (layer B.Cu) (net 1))
 (segment (start 65.025 100.575) (end 65.825 100.575) (width 0.2032) (layer B.Cu) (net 1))
 (segment (start 70.0837 103.05) (end 73.124 100.0097) (width 0.2032) (layer B.Cu) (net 1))
 (segment (start 68.3 103.05) (end 70.0837 103.05) (width 0.2032) (layer B.Cu) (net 1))
 (segment (start 81.125 102.825) (end 81.125 101.575) (width 0.2032) (layer B.Cu) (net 1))
 (segment (start 81.125 101.575) (end 80.85 101.3) (width 0.2032) (layer B.Cu) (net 1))
 (segment (start 79.524 100.0097) (end 79.524 99.0565) (width 0.2032) (layer B.Cu) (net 1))
 (segment (start 79.524 100.519225) (end 79.524 100.0097) (width 0.2032) (layer B.Cu) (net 1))
 (segment (start 80.304775 101.3) (end 79.524 100.519225) (width 0.2032) (layer B.Cu) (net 1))
 (segment (start 80.85 101.3) (end 80.304775 101.3) (width 0.2032) (layer B.Cu) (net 1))
 (segment (start 81.125 102.825) (end 81.125 103.625) (width 0.2032) (layer B.Cu) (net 1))
 (segment (start 79.524 98.1033) (end 77.9 96.4793) (width 0.2032) (layer B.Cu) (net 1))
 (segment (start 79.524 99.0565) (end 79.524 98.1033) (width 0.2032) (layer B.Cu) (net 1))
 (segment (start 77.9 96.4793) (end 77.9 90.875) (width 0.2032) (layer B.Cu) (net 1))
 (segment (start 79.4185 89.3565) (end 82.024 89.3565) (width 0.2032) (layer B.Cu) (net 1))
 (segment (start 77.9 90.875) (end 79.4185 89.3565) (width 0.2032) (layer B.Cu) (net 1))
 (segment (start 74.724 88.6097) (end 74.724 87.6565) (width 0.2032) (layer B.Cu) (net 1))
 (segment (start 76.9893 90.875) (end 74.724 88.6097) (width 0.2032) (layer B.Cu) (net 1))
 (segment (start 77.9 90.875) (end 76.9893 90.875) (width 0.2032) (layer B.Cu) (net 1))
 (segment (start 70.624 94.1565) (end 71.5815 94.1565) (width 0.2032) (layer B.Cu) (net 1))
 (segment (start 73.124 95.699) (end 73.124 99.0565) (width 0.2032) (layer B.Cu) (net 1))
 (segment (start 71.5815 94.1565) (end 73.124 95.699) (width 0.2032) (layer B.Cu) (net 1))
 (segment (start 77.1197 95.699) (end 77.9 96.4793) (width 0.2032) (layer B.Cu) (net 1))
 (segment (start 73.124 95.699) (end 77.1197 95.699) (width 0.2032) (layer B.Cu) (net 1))
 (segment (start 55.55 77.895) (end 58.055 80.4) (width 0.2032) (layer B.Cu) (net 1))
 (segment (start 55.55 77.02) (end 55.55 77.895) (width 0.2032) (layer B.Cu) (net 1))
 (segment (start 58.055 80.4) (end 58.055 92.555) (width 0.2032) (layer B.Cu) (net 1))
 (segment (start 58.055 92.555) (end 59.6565 94.1565) (width 0.2032) (layer B.Cu) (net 1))
 (segment (start 72.375 80.175) (end 71.575 80.175) (width 0.2032) (layer B.Cu) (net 1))
 (segment (start 77.042 78.564) (end 77.142 78.564) (width 0.2032) (layer B.Cu) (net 1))
 (segment (start 71.575 80.175) (end 70.075 78.675) (width 0.2032) (layer B.Cu) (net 1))
 (segment (start 70.075 78.675) (end 70.075 75.875) (width 0.2032) (layer B.Cu) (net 1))
 (segment (start 70.075 75.875) (end 70.55 75.4) (width 0.2032) (layer B.Cu) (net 1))
 (segment (start 70.55 75.4) (end 73.878 75.4) (width 0.2032) (layer B.Cu) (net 1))
 (segment (start 73.878 75.4) (end 77.042 78.564) (width 0.2032) (layer B.Cu) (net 1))
 (segment (start 79.711 78.564) (end 79.975 78.3) (width 0.2032) (layer B.Cu) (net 1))
 (segment (start 77.142 78.564) (end 79.711 78.564) (width 0.2032) (layer B.Cu) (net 1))
 (segment (start 74.724 86.7033) (end 74.724 87.6565) (width 0.2032) (layer B.Cu) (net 1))
 (segment (start 74.724 83.1115) (end 74.724 86.7033) (width 0.2032) (layer B.Cu) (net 1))
 (segment (start 72.375 80.7625) (end 74.724 83.1115) (width 0.2032) (layer B.Cu) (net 1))
 (segment (start 72.375 80.175) (end 72.375 80.7625) (width 0.2032) (layer B.Cu) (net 1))
 (segment (start 73.124 100.0097) (end 73.124 99.0565) (width 0.2032) (layer B.Cu) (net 1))
 (segment (start 73.025599 100.108101) (end 73.124 100.0097) (width 0.2032) (layer B.Cu) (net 1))
 (via (at 72.675 82.525) (size 0.8) (drill 0.4) (layers F.Cu B.Cu) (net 1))
 (segment (start 72.375 80.175) (end 72.375 82.225) (width 0.2032) (layer B.Cu) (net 1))
 (segment (start 72.375 82.225) (end 72.675 82.525) (width 0.2032) (layer B.Cu) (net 1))
 (via (at 76.35 82.55) (size 0.8) (drill 0.4) (layers F.Cu B.Cu) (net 1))
 (segment (start 72.675 82.525) (end 76.325 82.525) (width 0.2032) (layer F.Cu) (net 1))
 (segment (start 76.325 82.525) (end 76.35 82.55) (width 0.2032) (layer F.Cu) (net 1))
 (segment (start 75.042 80.264) (end 74.942 80.264) (width 0.2032) (layer B.Cu) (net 1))
 (segment (start 76.35 81.572) (end 75.042 80.264) (width 0.2032) (layer B.Cu) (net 1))
 (segment (start 76.35 82.55) (end 76.35 81.572) (width 0.2032) (layer B.Cu) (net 1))
 (segment (start 82.024 88.8783) (end 82.024 89.3565) (width 0.2032) (layer B.Cu) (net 1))
 (segment (start 82.4898 88.4125) (end 82.024 88.8783) (width 0.2032) (layer B.Cu) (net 1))
 (segment (start 85.55 88.4125) (end 82.4898 88.4125) (width 0.2032) (layer B.Cu) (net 1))
 (segment (start 62.5615 92.251) (end 62.5615 94.1565) (width 0.2032) (layer B.Cu) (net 1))
 (segment (start 63.5375 91.275) (end 62.5615 92.251) (width 0.2032) (layer B.Cu) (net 1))
 (segment (start 64.125 91.275) (end 63.5375 91.275) (width 0.2032) (layer B.Cu) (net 1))
 (segment (start 59.6565 94.1565) (end 62.5615 94.1565) (width 0.2032) (layer B.Cu) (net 1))
 (segment (start 86.2 100.325) (end 86.2 103.538) (width 0.2032) (layer B.Cu) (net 1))
 (segment (start 86.2 103.538) (end 85.09 104.648) (width 0.2032) (layer B.Cu) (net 1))
 (segment (start 82.948 104.648) (end 81.125 102.825) (width 0.2032) (layer B.Cu) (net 1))
 (segment (start 85.09 104.648) (end 82.948 104.648) (width 0.2032) (layer B.Cu) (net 1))
 (via (at 65.278 83.5484) (size 0.8) (drill 0.4) (layers F.Cu B.Cu) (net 1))
 (segment (start 65.3 82.6625) (end 65.3 83.5264) (width 0.2032) (layer B.Cu) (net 1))
 (segment (start 65.3 83.5264) (end 65.278 83.5484) (width 0.2032) (layer B.Cu) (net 1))
 (via (at 66.548 93.218) (size 0.8) (drill 0.4) (layers F.Cu B.Cu) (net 1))
 (segment (start 65.278 83.5484) (end 66.548 84.8184) (width 0.2032) (layer F.Cu) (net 1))
 (segment (start 66.548 84.8184) (end 66.548 93.218) (width 0.2032) (layer F.Cu) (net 1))
 (segment (start 68.311275 94.1565) (end 69.5185 94.1565) (width 0.2032) (layer B.Cu) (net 1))
 (segment (start 67.772774 93.617999) (end 68.311275 94.1565) (width 0.2032) (layer B.Cu) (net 1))
 (segment (start 66.947999 93.617999) (end 67.772774 93.617999) (width 0.2032) (layer B.Cu) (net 1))
 (segment (start 66.548 93.218) (end 66.947999 93.617999) (width 0.2032) (layer B.Cu) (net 1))
 (segment (start 62.5615 94.1565) (end 69.5185 94.1565) (width 0.2032) (layer B.Cu) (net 1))
 (segment (start 69.5185 94.1565) (end 70.624 94.1565) (width 0.2032) (layer B.Cu) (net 1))
 (segment (start 77.231 80.175) (end 77.142 80.264) (width 0.2032) (layer B.Cu) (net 3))
 (segment (start 79.975 80.175) (end 77.231 80.175) (width 0.2032) (layer B.Cu) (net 3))
 (segment (start 77.142 81.0672) (end 77.15 81.0752) (width 0.2032) (layer B.Cu) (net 3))
 (segment (start 77.142 80.264) (end 77.142 81.0672) (width 0.2032) (layer B.Cu) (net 3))
 (segment (start 77.15 81.0752) (end 77.15 84.4) (width 0.2032) (layer B.Cu) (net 3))
 (segment (start 76.324 85.226) (end 76.324 87.6565) (width 0.2032) (layer B.Cu) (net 3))
 (segment (start 77.15 84.4) (end 76.324 85.226) (width 0.2032) (layer B.Cu) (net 3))
 (segment (start 74.678 78.3) (end 74.942 78.564) (width 0.2032) (layer B.Cu) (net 4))
 (segment (start 72.375 78.3) (end 74.678 78.3) (width 0.2032) (layer B.Cu) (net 4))
 (segment (start 74.0388 78.564) (end 73.8 78.8028) (width 0.2032) (layer B.Cu) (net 4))
 (segment (start 74.942 78.564) (end 74.0388 78.564) (width 0.2032) (layer B.Cu) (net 4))
 (segment (start 75.524 86.7033) (end 75.524 87.6565) (width 0.2032) (layer B.Cu) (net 4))
 (segment (start 75.524 82.688882) (end 75.524 86.7033) (width 0.2032) (layer B.Cu) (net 4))
 (segment (start 73.8 80.964882) (end 75.524 82.688882) (width 0.2032) (layer B.Cu) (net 4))
 (segment (start 73.8 78.8028) (end 73.8 80.964882) (width 0.2032) (layer B.Cu) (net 4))
 (segment (start 68.0815 93.3565) (end 70.624 93.3565) (width 0.2032) (layer B.Cu) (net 5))
 (segment (start 66 91.275) (end 68.0815 93.3565) (width 0.2032) (layer B.Cu) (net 5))
 (segment (start 99.875 95.60775) (end 100.23275 95.60775) (width 0.2032) (layer B.Cu) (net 10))
 (segment (start 52.35 77.166139) (end 52.387946 77.030624) (width 0.2032) (layer B.Cu) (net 12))
 (segment (start 52.35 80.478742) (end 52.35 77.166139) (width 0.2032) (layer B.Cu) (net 12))
 (segment (start 47.13 89.29) (end 47.13 85.698742) (width 0.2032) (layer B.Cu) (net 12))
 (segment (start 47.13 85.698742) (end 52.35 80.478742) (width 0.2032) (layer B.Cu) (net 12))
 (segment (start 53.15 78.3482) (end 53.15 77.02) (width 0.2032) (layer B.Cu) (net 23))
 (segment (start 53.15 82.7) (end 53.15 77.02) (width 0.2032) (layer B.Cu) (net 23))
 (segment (start 52 83.85) (end 53.15 82.7) (width 0.2032) (layer B.Cu) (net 23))
 (segment (start 52 86.3125) (end 53.375 87.6875) (width 0.2032) (layer B.Cu) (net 24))
 (segment (start 52 85.725) (end 52 86.3125) (width 0.2032) (layer B.Cu) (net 24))
 (segment (start 53.375 87.6875) (end 53.375 91.475) (width 0.2032) (layer B.Cu) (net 24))
 (segment (start 57.6565 95.7565) (end 70.624 95.7565) (width 0.2032) (layer B.Cu) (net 24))
 (segment (start 53.375 91.475) (end 57.6565 95.7565) (width 0.2032) (layer B.Cu) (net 24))
 (segment (start 55.05 86.425) (end 54.025 87.45) (width 0.2032) (layer B.Cu) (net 25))
 (segment (start 55.05 85.8375) (end 55.05 86.425) (width 0.2032) (layer B.Cu) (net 25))
 (segment (start 54.025 87.45) (end 54.025 91.275) (width 0.2032) (layer B.Cu) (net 25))
 (segment (start 57.7065 94.9565) (end 70.624 94.9565) (width 0.2032) (layer B.Cu) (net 25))
 (segment (start 54.025 91.275) (end 57.7065 94.9565) (width 0.2032) (layer B.Cu) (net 25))
 (segment (start 53.95 82.8625) (end 55.05 83.9625) (width 0.2032) (layer B.Cu) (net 26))
 (segment (start 53.95 77.02) (end 53.95 82.8625) (width 0.2032) (layer B.Cu) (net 26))
 (segment (start 62 83.2375) (end 63.0125 84.25) (width 0.2032) (layer B.Cu) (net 27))
 (segment (start 62 82.65) (end 62 83.2375) (width 0.2032) (layer B.Cu) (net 27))
 (segment (start 73.124 86.7033) (end 73.124 87.6565) (width 0.2032) (layer B.Cu) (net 27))
 (segment (start 73.124 85.949) (end 73.124 86.7033) (width 0.2032) (layer B.Cu) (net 27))
 (segment (start 71.425 84.25) (end 73.124 85.949) (width 0.2032) (layer B.Cu) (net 27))
 (segment (start 63.0125 84.25) (end 71.425 84.25) (width 0.2032) (layer B.Cu) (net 27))
 (segment (start 56.6 99.375) (end 57.7032 99.375) (width 0.2032) (layer B.Cu) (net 27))
 (via (at 60.625 98.1) (size 0.8) (drill 0.4) (layers F.Cu B.Cu) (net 27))
 (segment (start 56.6 99.375) (end 59.35 99.375) (width 0.2032) (layer B.Cu) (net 27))
 (segment (start 59.35 99.375) (end 60.625 98.1) (width 0.2032) (layer B.Cu) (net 27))
 (via (at 61.1 86.125) (size 0.8) (drill 0.4) (layers F.Cu B.Cu) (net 27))
 (segment (start 60.625 98.1) (end 61.1 97.625) (width 0.2032) (layer F.Cu) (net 27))
 (segment (start 61.1 97.625) (end 61.1 86.125) (width 0.2032) (layer F.Cu) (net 27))
 (segment (start 61.1 83.55) (end 62 82.65) (width 0.2032) (layer B.Cu) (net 27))
 (segment (start 61.1 86.125) (end 61.1 83.55) (width 0.2032) (layer B.Cu) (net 27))
 (segment (start 85.1065 97.3565) (end 82.024 97.3565) (width 0.2032) (layer B.Cu) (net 28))
 (segment (start 86.2 98.45) (end 85.1065 97.3565) (width 0.2032) (layer B.Cu) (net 28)))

